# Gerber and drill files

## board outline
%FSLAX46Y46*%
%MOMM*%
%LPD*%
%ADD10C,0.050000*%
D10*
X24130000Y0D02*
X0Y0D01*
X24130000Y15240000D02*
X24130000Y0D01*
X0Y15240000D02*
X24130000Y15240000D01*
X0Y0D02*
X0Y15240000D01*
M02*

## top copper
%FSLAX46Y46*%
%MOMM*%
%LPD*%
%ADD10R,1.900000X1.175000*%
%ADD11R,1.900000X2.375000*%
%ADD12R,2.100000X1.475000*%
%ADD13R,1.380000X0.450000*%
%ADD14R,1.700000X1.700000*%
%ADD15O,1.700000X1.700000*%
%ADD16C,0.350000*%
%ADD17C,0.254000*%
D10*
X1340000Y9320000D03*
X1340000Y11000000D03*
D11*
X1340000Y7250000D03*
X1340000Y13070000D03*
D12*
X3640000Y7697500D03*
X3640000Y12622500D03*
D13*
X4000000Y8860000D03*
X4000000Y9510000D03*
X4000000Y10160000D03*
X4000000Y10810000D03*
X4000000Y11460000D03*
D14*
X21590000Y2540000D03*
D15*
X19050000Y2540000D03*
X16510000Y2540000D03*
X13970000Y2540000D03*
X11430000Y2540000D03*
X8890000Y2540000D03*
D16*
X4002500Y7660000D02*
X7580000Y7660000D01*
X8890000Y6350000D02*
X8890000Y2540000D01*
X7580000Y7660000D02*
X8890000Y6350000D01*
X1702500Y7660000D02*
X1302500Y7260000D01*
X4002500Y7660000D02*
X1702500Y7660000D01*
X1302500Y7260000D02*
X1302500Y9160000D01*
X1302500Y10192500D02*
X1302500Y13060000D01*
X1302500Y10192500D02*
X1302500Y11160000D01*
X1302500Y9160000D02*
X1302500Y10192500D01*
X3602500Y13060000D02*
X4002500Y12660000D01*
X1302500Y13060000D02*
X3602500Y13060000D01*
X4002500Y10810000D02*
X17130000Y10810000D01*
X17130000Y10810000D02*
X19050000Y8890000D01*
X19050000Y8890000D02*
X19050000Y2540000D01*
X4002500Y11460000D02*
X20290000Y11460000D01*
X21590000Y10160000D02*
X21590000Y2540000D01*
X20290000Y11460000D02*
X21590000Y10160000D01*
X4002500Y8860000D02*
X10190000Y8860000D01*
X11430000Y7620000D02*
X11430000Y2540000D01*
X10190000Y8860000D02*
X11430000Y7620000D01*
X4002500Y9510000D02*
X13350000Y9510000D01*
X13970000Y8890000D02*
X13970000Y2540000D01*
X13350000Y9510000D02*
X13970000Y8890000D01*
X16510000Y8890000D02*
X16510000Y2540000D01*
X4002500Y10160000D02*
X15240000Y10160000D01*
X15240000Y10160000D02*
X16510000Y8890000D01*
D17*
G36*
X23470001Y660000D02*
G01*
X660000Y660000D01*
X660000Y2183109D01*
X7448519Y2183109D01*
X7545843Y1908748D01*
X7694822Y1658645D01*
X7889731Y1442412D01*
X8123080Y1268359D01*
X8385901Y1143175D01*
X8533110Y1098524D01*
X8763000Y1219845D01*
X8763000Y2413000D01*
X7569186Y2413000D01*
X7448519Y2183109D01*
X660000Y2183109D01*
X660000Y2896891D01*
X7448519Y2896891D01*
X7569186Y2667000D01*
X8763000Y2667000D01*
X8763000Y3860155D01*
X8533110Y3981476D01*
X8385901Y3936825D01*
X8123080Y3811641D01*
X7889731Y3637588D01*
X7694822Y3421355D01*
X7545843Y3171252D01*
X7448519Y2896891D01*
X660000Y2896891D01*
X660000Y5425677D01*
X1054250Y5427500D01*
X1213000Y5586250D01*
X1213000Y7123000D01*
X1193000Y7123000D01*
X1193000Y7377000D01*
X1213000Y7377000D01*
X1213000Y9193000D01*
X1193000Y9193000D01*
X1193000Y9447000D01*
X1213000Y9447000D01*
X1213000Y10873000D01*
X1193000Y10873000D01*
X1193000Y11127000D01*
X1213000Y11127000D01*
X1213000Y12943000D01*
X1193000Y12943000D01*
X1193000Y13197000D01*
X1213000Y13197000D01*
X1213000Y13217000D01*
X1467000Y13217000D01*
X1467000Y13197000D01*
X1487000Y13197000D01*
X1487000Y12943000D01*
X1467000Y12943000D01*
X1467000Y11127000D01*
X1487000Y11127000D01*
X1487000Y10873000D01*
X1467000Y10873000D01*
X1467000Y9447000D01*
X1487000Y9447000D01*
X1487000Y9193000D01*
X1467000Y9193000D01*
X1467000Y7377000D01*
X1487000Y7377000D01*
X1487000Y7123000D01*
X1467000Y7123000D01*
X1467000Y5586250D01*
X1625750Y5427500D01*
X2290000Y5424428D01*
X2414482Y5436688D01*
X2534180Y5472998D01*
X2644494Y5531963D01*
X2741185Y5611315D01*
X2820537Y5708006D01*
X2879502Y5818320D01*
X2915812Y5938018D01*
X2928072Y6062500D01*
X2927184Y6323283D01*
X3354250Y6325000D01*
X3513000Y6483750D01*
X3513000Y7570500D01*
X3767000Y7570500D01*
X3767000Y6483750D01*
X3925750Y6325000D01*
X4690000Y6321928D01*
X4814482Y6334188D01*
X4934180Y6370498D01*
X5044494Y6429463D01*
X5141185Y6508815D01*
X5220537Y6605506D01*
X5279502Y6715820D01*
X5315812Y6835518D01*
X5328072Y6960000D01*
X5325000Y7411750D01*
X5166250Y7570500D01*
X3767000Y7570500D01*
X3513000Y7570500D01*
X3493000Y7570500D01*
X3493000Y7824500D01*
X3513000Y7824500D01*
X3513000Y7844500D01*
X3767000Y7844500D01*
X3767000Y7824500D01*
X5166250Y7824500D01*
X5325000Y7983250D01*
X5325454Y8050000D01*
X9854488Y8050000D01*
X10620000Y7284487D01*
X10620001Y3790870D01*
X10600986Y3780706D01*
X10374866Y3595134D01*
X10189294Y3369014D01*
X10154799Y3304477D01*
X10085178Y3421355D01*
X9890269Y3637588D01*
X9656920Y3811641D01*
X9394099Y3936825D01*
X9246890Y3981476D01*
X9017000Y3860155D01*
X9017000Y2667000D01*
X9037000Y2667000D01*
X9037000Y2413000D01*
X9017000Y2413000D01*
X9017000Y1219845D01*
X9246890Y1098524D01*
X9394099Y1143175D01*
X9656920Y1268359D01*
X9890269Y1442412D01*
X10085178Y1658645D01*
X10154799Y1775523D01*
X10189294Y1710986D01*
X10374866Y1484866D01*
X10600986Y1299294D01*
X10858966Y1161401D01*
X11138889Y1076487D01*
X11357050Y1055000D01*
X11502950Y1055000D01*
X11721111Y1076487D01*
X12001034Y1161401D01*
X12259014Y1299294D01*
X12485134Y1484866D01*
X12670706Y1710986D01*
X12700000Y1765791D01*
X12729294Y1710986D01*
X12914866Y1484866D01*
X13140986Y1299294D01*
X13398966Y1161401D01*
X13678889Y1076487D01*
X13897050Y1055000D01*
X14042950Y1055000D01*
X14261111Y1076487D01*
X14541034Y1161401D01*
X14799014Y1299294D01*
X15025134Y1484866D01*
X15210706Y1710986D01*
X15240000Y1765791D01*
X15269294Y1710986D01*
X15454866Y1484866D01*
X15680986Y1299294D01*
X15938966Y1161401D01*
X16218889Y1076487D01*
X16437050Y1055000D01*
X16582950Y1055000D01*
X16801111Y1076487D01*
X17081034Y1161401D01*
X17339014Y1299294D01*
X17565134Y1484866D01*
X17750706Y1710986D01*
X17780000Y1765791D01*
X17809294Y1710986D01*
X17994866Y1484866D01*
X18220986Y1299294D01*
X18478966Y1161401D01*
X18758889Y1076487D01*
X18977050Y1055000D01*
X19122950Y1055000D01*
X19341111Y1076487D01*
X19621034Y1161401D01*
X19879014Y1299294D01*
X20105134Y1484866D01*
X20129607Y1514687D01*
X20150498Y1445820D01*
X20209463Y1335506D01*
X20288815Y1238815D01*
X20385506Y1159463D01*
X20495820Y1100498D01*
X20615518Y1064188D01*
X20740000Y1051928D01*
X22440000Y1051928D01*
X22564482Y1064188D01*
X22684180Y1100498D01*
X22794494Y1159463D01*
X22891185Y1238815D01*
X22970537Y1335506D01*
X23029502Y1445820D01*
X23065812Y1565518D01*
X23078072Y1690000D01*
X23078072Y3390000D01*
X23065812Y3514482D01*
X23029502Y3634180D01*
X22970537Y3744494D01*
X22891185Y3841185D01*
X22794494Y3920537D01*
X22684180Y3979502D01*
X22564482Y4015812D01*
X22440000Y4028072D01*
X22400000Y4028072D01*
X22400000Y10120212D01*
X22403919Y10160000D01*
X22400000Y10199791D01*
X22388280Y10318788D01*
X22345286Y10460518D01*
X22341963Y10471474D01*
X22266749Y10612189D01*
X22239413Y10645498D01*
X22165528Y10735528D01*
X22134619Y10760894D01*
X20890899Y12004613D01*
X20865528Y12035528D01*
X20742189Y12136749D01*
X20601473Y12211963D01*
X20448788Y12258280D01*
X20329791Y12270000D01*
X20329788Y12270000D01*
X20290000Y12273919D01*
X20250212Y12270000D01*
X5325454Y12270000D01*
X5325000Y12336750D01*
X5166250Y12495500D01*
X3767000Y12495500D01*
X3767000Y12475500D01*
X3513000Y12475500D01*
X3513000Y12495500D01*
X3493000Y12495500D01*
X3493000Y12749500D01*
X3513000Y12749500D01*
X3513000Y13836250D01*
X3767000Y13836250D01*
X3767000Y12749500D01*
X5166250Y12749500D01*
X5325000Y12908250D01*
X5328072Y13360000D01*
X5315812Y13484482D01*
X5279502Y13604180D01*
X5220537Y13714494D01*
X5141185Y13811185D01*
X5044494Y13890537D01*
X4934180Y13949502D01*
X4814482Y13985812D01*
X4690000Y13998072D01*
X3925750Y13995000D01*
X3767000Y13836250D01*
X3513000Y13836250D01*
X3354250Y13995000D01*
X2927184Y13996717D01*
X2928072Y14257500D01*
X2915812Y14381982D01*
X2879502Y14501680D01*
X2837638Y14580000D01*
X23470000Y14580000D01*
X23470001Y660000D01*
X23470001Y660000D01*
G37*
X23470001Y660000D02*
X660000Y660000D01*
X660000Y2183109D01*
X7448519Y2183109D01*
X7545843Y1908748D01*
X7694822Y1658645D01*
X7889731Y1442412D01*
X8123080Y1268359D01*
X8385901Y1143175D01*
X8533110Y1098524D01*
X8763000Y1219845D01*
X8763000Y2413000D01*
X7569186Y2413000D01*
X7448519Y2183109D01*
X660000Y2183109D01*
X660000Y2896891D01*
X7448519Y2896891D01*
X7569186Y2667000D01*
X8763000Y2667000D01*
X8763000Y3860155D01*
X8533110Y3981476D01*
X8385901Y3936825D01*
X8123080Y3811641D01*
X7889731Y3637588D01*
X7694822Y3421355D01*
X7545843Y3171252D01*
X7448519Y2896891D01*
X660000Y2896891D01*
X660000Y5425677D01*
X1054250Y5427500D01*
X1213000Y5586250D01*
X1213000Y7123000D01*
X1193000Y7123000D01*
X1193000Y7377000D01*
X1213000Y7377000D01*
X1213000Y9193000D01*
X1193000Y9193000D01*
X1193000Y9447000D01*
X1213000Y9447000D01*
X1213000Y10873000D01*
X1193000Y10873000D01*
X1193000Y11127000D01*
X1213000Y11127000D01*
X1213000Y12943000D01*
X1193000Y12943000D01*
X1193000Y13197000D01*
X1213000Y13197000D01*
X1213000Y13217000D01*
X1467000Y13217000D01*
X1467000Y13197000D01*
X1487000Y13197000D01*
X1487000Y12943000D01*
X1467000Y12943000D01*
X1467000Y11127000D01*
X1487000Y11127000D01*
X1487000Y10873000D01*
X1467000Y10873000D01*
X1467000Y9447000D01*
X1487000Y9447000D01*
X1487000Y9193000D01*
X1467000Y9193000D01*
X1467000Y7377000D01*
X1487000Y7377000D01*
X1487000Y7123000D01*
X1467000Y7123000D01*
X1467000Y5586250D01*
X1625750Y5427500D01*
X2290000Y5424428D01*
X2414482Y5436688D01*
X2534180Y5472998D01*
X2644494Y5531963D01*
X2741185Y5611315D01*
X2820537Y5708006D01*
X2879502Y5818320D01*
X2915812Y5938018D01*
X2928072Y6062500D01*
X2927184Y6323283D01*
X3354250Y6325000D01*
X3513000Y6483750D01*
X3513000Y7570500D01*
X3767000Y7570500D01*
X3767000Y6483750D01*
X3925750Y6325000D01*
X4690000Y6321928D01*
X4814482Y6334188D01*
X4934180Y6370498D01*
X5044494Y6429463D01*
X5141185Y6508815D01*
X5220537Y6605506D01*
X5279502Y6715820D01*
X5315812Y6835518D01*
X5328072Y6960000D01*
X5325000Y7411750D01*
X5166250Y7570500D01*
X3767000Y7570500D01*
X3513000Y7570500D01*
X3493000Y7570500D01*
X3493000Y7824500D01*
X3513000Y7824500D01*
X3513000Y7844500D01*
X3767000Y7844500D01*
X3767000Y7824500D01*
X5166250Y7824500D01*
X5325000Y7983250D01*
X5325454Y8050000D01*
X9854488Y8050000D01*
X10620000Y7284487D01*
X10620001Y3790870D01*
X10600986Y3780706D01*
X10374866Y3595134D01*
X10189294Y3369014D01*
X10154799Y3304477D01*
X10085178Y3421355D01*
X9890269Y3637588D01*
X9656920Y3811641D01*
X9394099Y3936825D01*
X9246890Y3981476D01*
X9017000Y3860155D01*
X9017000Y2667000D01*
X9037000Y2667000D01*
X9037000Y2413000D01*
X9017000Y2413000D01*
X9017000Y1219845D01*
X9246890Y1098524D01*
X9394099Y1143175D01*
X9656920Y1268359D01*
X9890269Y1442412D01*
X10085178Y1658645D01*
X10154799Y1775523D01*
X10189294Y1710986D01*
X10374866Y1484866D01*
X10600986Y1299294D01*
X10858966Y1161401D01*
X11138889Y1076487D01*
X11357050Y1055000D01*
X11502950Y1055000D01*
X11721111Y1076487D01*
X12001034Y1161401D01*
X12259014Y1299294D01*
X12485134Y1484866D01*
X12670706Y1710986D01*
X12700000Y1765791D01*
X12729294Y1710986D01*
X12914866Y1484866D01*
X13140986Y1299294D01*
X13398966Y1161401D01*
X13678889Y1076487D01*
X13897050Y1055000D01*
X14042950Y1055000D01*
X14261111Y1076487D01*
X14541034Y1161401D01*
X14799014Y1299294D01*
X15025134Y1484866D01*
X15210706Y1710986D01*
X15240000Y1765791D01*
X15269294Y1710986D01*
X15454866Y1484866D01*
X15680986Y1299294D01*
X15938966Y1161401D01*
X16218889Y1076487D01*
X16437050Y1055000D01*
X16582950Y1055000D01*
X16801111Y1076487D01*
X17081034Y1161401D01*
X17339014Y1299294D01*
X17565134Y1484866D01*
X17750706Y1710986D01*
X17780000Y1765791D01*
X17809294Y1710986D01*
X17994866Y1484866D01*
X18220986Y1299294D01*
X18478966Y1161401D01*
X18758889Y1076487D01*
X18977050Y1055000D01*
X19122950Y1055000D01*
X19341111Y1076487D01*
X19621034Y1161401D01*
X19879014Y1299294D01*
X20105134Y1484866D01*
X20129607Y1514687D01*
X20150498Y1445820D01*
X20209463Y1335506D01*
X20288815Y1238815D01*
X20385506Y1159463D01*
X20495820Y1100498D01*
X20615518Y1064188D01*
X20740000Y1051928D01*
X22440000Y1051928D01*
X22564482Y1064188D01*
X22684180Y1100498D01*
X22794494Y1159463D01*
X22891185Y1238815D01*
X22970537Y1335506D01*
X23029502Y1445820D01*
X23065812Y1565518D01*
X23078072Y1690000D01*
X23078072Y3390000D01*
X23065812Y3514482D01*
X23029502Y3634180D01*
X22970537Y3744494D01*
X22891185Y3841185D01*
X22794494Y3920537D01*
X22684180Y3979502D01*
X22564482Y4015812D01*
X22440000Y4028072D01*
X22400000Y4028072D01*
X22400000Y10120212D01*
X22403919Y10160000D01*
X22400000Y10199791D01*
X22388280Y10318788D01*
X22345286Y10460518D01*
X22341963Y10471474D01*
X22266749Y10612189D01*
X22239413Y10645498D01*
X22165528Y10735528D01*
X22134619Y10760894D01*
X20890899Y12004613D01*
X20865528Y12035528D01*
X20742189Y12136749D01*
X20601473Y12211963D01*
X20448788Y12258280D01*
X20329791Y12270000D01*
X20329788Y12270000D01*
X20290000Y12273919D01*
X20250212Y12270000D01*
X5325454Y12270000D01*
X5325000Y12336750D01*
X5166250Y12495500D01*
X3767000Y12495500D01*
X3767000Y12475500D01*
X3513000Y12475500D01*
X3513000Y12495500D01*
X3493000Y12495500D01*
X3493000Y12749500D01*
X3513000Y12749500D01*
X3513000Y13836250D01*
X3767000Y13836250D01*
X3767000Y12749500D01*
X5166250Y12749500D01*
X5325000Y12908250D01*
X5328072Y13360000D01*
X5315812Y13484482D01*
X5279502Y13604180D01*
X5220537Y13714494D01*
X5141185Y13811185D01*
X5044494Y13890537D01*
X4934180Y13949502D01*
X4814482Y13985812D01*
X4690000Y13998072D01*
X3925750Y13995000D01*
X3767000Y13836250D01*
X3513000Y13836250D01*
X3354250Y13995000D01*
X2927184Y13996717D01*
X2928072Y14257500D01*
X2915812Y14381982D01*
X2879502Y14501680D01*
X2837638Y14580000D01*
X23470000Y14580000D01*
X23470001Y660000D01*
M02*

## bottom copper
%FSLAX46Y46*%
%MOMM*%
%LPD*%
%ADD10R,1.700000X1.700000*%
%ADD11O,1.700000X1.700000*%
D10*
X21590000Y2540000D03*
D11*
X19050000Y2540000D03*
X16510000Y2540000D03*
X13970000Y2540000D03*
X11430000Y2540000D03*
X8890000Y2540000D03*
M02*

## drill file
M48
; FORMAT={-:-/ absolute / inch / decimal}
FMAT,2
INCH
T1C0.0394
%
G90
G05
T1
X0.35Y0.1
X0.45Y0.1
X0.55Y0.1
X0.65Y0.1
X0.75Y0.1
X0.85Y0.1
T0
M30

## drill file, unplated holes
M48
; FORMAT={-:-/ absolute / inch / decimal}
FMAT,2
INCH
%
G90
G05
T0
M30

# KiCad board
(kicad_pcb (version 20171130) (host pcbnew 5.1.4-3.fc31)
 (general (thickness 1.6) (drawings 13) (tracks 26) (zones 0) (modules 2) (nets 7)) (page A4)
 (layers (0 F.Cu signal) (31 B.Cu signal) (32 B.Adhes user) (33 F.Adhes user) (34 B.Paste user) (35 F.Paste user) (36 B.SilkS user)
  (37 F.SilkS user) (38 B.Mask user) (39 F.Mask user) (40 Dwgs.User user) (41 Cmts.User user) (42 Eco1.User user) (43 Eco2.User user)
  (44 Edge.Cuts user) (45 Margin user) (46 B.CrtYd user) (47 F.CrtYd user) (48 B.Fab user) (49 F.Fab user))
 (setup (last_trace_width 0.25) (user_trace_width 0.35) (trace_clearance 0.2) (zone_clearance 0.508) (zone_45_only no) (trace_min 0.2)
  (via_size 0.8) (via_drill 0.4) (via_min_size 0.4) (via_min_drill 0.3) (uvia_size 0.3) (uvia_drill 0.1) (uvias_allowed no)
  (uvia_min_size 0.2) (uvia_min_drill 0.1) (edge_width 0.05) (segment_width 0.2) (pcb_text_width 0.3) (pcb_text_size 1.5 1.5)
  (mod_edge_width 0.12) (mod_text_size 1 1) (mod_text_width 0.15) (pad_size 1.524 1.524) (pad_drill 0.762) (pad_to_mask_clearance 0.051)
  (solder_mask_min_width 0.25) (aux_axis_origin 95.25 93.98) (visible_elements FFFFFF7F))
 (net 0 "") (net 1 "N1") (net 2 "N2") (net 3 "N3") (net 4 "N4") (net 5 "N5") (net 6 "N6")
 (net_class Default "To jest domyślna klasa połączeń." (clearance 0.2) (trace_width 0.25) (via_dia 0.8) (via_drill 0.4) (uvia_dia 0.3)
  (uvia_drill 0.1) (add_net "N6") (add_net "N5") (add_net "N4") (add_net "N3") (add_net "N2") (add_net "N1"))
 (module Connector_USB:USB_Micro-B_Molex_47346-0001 (layer F.Cu) (at 97.79 83.82 270)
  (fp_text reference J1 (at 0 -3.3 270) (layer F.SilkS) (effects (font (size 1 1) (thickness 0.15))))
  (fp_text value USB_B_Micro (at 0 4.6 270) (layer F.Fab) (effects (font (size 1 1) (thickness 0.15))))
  (pad 6 smd rect (at 0.84 1.2 270) (size 1.175 1.9) (layers F.Cu F.Paste F.Mask) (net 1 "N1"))
  (pad 6 smd rect (at -0.84 1.2 270) (size 1.175 1.9) (layers F.Cu F.Paste F.Mask) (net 1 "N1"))
  (pad 6 smd rect (at 2.91 1.2 270) (size 2.375 1.9) (layers F.Cu F.Paste F.Mask) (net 1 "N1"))
  (pad 6 smd rect (at -2.91 1.2 270) (size 2.375 1.9) (layers F.Cu F.Paste F.Mask) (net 1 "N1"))
  (pad 6 smd rect (at 2.4625 -1.1 270) (size 1.475 2.1) (layers F.Cu F.Paste F.Mask) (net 1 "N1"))
  (pad 6 smd rect (at -2.4625 -1.1 270) (size 1.475 2.1) (layers F.Cu F.Paste F.Mask) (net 1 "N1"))
  (pad 5 smd rect (at 1.3 -1.46 270) (size 0.45 1.38) (layers F.Cu F.Paste F.Mask) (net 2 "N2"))
  (pad 4 smd rect (at 0.65 -1.46 270) (size 0.45 1.38) (layers F.Cu F.Paste F.Mask) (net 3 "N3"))
  (pad 3 smd rect (at 0 -1.46 270) (size 0.45 1.38) (layers F.Cu F.Paste F.Mask) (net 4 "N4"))
  (pad 2 smd rect (at -0.65 -1.46 270) (size 0.45 1.38) (layers F.Cu F.Paste F.Mask) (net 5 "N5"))
  (pad 1 smd rect (at -1.3 -1.46 270) (size 0.45 1.38) (layers F.Cu F.Paste F.Mask) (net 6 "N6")))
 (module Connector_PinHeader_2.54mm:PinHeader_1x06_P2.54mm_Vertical (layer B.Cu) (at 116.84 91.44 90)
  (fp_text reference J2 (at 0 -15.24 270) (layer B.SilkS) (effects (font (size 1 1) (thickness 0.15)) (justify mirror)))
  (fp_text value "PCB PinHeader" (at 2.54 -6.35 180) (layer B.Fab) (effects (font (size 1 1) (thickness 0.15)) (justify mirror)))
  (pad 1 thru_hole rect (at 0 0 90) (size 1.7 1.7) (drill 1) (layers *.Cu *.Mask) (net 6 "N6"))
  (pad 2 thru_hole oval (at 0 -2.54 90) (size 1.7 1.7) (drill 1) (layers *.Cu *.Mask) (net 5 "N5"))
  (pad 3 thru_hole oval (at 0 -5.08 90) (size 1.7 1.7) (drill 1) (layers *.Cu *.Mask) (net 4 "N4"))
  (pad 4 thru_hole oval (at 0 -7.62 90) (size 1.7 1.7) (drill 1) (layers *.Cu *.Mask) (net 3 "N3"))
  (pad 5 thru_hole oval (at 0 -10.16 90) (size 1.7 1.7) (drill 1) (layers *.Cu *.Mask) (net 2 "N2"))
  (pad 6 thru_hole oval (at 0 -12.7 90) (size 1.7 1.7) (drill 1) (layers *.Cu *.Mask) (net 1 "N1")))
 (gr_line (start 119.38 93.98) (end 95.25 93.98) (layer Edge.Cuts) (width 0.05))
 (gr_line (start 119.38 78.74) (end 119.38 93.98) (layer Edge.Cuts) (width 0.05))
 (gr_line (start 95.25 78.74) (end 119.38 78.74) (layer Edge.Cuts) (width 0.05))
 (gr_line (start 95.25 93.98) (end 95.25 78.74) (layer Edge.Cuts) (width 0.05))
 (segment (start 99.2525 86.32) (end 102.83 86.32) (width 0.35) (layer F.Cu) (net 1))
 (segment (start 104.14 87.63) (end 104.14 91.44) (width 0.35) (layer F.Cu) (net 1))
 (segment (start 102.83 86.32) (end 104.14 87.63) (width 0.35) (layer F.Cu) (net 1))
 (segment (start 96.9525 86.32) (end 96.5525 86.72) (width 0.35) (layer F.Cu) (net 1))
 (segment (start 99.2525 86.32) (end 96.9525 86.32) (width 0.35) (layer F.Cu) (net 1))
 (segment (start 96.5525 86.72) (end 96.5525 84.82) (width 0.35) (layer F.Cu) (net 1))
 (segment (start 96.5525 83.7875) (end 96.5525 80.92) (width 0.35) (layer F.Cu) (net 1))
 (segment (start 96.5525 83.7875) (end 96.5525 82.82) (width 0.35) (layer F.Cu) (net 1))
 (segment (start 96.5525 84.82) (end 96.5525 83.7875) (width 0.35) (layer F.Cu) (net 1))
 (segment (start 98.8525 80.92) (end 99.2525 81.32) (width 0.35) (layer F.Cu) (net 1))
 (segment (start 96.5525 80.92) (end 98.8525 80.92) (width 0.35) (layer F.Cu) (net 1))
 (segment (start 99.2525 83.17) (end 112.38 83.17) (width 0.35) (layer F.Cu) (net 5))
 (segment (start 112.38 83.17) (end 114.3 85.09) (width 0.35) (layer F.Cu) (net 5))
 (segment (start 114.3 85.09) (end 114.3 91.44) (width 0.35) (layer F.Cu) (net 5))
 (segment (start 99.2525 82.52) (end 115.54 82.52) (width 0.35) (layer F.Cu) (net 6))
 (segment (start 116.84 83.82) (end 116.84 91.44) (width 0.35) (layer F.Cu) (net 6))
 (segment (start 115.54 82.52) (end 116.84 83.82) (width 0.35) (layer F.Cu) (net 6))
 (segment (start 99.2525 85.12) (end 105.44 85.12) (width 0.35) (layer F.Cu) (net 2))
 (segment (start 106.68 86.36) (end 106.68 91.44) (width 0.35) (layer F.Cu) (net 2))
 (segment (start 105.44 85.12) (end 106.68 86.36) (width 0.35) (layer F.Cu) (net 2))
 (segment (start 99.2525 84.47) (end 108.6 84.47) (width 0.35) (layer F.Cu) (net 3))
 (segment (start 109.22 85.09) (end 109.22 91.44) (width 0.35) (layer F.Cu) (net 3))
 (segment (start 108.6 84.47) (end 109.22 85.09) (width 0.35) (layer F.Cu) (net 3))
 (segment (start 111.76 85.09) (end 111.76 91.44) (width 0.35) (layer F.Cu) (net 4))
 (segment (start 99.2525 83.82) (end 110.49 83.82) (width 0.35) (layer F.Cu) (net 4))
 (segment (start 110.49 83.82) (end 111.76 85.09) (width 0.35) (layer F.Cu) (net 4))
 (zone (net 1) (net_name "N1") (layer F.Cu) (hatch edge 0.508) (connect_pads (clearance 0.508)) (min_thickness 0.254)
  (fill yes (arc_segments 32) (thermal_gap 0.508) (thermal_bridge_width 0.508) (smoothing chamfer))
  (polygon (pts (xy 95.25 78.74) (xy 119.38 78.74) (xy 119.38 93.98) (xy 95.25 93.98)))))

